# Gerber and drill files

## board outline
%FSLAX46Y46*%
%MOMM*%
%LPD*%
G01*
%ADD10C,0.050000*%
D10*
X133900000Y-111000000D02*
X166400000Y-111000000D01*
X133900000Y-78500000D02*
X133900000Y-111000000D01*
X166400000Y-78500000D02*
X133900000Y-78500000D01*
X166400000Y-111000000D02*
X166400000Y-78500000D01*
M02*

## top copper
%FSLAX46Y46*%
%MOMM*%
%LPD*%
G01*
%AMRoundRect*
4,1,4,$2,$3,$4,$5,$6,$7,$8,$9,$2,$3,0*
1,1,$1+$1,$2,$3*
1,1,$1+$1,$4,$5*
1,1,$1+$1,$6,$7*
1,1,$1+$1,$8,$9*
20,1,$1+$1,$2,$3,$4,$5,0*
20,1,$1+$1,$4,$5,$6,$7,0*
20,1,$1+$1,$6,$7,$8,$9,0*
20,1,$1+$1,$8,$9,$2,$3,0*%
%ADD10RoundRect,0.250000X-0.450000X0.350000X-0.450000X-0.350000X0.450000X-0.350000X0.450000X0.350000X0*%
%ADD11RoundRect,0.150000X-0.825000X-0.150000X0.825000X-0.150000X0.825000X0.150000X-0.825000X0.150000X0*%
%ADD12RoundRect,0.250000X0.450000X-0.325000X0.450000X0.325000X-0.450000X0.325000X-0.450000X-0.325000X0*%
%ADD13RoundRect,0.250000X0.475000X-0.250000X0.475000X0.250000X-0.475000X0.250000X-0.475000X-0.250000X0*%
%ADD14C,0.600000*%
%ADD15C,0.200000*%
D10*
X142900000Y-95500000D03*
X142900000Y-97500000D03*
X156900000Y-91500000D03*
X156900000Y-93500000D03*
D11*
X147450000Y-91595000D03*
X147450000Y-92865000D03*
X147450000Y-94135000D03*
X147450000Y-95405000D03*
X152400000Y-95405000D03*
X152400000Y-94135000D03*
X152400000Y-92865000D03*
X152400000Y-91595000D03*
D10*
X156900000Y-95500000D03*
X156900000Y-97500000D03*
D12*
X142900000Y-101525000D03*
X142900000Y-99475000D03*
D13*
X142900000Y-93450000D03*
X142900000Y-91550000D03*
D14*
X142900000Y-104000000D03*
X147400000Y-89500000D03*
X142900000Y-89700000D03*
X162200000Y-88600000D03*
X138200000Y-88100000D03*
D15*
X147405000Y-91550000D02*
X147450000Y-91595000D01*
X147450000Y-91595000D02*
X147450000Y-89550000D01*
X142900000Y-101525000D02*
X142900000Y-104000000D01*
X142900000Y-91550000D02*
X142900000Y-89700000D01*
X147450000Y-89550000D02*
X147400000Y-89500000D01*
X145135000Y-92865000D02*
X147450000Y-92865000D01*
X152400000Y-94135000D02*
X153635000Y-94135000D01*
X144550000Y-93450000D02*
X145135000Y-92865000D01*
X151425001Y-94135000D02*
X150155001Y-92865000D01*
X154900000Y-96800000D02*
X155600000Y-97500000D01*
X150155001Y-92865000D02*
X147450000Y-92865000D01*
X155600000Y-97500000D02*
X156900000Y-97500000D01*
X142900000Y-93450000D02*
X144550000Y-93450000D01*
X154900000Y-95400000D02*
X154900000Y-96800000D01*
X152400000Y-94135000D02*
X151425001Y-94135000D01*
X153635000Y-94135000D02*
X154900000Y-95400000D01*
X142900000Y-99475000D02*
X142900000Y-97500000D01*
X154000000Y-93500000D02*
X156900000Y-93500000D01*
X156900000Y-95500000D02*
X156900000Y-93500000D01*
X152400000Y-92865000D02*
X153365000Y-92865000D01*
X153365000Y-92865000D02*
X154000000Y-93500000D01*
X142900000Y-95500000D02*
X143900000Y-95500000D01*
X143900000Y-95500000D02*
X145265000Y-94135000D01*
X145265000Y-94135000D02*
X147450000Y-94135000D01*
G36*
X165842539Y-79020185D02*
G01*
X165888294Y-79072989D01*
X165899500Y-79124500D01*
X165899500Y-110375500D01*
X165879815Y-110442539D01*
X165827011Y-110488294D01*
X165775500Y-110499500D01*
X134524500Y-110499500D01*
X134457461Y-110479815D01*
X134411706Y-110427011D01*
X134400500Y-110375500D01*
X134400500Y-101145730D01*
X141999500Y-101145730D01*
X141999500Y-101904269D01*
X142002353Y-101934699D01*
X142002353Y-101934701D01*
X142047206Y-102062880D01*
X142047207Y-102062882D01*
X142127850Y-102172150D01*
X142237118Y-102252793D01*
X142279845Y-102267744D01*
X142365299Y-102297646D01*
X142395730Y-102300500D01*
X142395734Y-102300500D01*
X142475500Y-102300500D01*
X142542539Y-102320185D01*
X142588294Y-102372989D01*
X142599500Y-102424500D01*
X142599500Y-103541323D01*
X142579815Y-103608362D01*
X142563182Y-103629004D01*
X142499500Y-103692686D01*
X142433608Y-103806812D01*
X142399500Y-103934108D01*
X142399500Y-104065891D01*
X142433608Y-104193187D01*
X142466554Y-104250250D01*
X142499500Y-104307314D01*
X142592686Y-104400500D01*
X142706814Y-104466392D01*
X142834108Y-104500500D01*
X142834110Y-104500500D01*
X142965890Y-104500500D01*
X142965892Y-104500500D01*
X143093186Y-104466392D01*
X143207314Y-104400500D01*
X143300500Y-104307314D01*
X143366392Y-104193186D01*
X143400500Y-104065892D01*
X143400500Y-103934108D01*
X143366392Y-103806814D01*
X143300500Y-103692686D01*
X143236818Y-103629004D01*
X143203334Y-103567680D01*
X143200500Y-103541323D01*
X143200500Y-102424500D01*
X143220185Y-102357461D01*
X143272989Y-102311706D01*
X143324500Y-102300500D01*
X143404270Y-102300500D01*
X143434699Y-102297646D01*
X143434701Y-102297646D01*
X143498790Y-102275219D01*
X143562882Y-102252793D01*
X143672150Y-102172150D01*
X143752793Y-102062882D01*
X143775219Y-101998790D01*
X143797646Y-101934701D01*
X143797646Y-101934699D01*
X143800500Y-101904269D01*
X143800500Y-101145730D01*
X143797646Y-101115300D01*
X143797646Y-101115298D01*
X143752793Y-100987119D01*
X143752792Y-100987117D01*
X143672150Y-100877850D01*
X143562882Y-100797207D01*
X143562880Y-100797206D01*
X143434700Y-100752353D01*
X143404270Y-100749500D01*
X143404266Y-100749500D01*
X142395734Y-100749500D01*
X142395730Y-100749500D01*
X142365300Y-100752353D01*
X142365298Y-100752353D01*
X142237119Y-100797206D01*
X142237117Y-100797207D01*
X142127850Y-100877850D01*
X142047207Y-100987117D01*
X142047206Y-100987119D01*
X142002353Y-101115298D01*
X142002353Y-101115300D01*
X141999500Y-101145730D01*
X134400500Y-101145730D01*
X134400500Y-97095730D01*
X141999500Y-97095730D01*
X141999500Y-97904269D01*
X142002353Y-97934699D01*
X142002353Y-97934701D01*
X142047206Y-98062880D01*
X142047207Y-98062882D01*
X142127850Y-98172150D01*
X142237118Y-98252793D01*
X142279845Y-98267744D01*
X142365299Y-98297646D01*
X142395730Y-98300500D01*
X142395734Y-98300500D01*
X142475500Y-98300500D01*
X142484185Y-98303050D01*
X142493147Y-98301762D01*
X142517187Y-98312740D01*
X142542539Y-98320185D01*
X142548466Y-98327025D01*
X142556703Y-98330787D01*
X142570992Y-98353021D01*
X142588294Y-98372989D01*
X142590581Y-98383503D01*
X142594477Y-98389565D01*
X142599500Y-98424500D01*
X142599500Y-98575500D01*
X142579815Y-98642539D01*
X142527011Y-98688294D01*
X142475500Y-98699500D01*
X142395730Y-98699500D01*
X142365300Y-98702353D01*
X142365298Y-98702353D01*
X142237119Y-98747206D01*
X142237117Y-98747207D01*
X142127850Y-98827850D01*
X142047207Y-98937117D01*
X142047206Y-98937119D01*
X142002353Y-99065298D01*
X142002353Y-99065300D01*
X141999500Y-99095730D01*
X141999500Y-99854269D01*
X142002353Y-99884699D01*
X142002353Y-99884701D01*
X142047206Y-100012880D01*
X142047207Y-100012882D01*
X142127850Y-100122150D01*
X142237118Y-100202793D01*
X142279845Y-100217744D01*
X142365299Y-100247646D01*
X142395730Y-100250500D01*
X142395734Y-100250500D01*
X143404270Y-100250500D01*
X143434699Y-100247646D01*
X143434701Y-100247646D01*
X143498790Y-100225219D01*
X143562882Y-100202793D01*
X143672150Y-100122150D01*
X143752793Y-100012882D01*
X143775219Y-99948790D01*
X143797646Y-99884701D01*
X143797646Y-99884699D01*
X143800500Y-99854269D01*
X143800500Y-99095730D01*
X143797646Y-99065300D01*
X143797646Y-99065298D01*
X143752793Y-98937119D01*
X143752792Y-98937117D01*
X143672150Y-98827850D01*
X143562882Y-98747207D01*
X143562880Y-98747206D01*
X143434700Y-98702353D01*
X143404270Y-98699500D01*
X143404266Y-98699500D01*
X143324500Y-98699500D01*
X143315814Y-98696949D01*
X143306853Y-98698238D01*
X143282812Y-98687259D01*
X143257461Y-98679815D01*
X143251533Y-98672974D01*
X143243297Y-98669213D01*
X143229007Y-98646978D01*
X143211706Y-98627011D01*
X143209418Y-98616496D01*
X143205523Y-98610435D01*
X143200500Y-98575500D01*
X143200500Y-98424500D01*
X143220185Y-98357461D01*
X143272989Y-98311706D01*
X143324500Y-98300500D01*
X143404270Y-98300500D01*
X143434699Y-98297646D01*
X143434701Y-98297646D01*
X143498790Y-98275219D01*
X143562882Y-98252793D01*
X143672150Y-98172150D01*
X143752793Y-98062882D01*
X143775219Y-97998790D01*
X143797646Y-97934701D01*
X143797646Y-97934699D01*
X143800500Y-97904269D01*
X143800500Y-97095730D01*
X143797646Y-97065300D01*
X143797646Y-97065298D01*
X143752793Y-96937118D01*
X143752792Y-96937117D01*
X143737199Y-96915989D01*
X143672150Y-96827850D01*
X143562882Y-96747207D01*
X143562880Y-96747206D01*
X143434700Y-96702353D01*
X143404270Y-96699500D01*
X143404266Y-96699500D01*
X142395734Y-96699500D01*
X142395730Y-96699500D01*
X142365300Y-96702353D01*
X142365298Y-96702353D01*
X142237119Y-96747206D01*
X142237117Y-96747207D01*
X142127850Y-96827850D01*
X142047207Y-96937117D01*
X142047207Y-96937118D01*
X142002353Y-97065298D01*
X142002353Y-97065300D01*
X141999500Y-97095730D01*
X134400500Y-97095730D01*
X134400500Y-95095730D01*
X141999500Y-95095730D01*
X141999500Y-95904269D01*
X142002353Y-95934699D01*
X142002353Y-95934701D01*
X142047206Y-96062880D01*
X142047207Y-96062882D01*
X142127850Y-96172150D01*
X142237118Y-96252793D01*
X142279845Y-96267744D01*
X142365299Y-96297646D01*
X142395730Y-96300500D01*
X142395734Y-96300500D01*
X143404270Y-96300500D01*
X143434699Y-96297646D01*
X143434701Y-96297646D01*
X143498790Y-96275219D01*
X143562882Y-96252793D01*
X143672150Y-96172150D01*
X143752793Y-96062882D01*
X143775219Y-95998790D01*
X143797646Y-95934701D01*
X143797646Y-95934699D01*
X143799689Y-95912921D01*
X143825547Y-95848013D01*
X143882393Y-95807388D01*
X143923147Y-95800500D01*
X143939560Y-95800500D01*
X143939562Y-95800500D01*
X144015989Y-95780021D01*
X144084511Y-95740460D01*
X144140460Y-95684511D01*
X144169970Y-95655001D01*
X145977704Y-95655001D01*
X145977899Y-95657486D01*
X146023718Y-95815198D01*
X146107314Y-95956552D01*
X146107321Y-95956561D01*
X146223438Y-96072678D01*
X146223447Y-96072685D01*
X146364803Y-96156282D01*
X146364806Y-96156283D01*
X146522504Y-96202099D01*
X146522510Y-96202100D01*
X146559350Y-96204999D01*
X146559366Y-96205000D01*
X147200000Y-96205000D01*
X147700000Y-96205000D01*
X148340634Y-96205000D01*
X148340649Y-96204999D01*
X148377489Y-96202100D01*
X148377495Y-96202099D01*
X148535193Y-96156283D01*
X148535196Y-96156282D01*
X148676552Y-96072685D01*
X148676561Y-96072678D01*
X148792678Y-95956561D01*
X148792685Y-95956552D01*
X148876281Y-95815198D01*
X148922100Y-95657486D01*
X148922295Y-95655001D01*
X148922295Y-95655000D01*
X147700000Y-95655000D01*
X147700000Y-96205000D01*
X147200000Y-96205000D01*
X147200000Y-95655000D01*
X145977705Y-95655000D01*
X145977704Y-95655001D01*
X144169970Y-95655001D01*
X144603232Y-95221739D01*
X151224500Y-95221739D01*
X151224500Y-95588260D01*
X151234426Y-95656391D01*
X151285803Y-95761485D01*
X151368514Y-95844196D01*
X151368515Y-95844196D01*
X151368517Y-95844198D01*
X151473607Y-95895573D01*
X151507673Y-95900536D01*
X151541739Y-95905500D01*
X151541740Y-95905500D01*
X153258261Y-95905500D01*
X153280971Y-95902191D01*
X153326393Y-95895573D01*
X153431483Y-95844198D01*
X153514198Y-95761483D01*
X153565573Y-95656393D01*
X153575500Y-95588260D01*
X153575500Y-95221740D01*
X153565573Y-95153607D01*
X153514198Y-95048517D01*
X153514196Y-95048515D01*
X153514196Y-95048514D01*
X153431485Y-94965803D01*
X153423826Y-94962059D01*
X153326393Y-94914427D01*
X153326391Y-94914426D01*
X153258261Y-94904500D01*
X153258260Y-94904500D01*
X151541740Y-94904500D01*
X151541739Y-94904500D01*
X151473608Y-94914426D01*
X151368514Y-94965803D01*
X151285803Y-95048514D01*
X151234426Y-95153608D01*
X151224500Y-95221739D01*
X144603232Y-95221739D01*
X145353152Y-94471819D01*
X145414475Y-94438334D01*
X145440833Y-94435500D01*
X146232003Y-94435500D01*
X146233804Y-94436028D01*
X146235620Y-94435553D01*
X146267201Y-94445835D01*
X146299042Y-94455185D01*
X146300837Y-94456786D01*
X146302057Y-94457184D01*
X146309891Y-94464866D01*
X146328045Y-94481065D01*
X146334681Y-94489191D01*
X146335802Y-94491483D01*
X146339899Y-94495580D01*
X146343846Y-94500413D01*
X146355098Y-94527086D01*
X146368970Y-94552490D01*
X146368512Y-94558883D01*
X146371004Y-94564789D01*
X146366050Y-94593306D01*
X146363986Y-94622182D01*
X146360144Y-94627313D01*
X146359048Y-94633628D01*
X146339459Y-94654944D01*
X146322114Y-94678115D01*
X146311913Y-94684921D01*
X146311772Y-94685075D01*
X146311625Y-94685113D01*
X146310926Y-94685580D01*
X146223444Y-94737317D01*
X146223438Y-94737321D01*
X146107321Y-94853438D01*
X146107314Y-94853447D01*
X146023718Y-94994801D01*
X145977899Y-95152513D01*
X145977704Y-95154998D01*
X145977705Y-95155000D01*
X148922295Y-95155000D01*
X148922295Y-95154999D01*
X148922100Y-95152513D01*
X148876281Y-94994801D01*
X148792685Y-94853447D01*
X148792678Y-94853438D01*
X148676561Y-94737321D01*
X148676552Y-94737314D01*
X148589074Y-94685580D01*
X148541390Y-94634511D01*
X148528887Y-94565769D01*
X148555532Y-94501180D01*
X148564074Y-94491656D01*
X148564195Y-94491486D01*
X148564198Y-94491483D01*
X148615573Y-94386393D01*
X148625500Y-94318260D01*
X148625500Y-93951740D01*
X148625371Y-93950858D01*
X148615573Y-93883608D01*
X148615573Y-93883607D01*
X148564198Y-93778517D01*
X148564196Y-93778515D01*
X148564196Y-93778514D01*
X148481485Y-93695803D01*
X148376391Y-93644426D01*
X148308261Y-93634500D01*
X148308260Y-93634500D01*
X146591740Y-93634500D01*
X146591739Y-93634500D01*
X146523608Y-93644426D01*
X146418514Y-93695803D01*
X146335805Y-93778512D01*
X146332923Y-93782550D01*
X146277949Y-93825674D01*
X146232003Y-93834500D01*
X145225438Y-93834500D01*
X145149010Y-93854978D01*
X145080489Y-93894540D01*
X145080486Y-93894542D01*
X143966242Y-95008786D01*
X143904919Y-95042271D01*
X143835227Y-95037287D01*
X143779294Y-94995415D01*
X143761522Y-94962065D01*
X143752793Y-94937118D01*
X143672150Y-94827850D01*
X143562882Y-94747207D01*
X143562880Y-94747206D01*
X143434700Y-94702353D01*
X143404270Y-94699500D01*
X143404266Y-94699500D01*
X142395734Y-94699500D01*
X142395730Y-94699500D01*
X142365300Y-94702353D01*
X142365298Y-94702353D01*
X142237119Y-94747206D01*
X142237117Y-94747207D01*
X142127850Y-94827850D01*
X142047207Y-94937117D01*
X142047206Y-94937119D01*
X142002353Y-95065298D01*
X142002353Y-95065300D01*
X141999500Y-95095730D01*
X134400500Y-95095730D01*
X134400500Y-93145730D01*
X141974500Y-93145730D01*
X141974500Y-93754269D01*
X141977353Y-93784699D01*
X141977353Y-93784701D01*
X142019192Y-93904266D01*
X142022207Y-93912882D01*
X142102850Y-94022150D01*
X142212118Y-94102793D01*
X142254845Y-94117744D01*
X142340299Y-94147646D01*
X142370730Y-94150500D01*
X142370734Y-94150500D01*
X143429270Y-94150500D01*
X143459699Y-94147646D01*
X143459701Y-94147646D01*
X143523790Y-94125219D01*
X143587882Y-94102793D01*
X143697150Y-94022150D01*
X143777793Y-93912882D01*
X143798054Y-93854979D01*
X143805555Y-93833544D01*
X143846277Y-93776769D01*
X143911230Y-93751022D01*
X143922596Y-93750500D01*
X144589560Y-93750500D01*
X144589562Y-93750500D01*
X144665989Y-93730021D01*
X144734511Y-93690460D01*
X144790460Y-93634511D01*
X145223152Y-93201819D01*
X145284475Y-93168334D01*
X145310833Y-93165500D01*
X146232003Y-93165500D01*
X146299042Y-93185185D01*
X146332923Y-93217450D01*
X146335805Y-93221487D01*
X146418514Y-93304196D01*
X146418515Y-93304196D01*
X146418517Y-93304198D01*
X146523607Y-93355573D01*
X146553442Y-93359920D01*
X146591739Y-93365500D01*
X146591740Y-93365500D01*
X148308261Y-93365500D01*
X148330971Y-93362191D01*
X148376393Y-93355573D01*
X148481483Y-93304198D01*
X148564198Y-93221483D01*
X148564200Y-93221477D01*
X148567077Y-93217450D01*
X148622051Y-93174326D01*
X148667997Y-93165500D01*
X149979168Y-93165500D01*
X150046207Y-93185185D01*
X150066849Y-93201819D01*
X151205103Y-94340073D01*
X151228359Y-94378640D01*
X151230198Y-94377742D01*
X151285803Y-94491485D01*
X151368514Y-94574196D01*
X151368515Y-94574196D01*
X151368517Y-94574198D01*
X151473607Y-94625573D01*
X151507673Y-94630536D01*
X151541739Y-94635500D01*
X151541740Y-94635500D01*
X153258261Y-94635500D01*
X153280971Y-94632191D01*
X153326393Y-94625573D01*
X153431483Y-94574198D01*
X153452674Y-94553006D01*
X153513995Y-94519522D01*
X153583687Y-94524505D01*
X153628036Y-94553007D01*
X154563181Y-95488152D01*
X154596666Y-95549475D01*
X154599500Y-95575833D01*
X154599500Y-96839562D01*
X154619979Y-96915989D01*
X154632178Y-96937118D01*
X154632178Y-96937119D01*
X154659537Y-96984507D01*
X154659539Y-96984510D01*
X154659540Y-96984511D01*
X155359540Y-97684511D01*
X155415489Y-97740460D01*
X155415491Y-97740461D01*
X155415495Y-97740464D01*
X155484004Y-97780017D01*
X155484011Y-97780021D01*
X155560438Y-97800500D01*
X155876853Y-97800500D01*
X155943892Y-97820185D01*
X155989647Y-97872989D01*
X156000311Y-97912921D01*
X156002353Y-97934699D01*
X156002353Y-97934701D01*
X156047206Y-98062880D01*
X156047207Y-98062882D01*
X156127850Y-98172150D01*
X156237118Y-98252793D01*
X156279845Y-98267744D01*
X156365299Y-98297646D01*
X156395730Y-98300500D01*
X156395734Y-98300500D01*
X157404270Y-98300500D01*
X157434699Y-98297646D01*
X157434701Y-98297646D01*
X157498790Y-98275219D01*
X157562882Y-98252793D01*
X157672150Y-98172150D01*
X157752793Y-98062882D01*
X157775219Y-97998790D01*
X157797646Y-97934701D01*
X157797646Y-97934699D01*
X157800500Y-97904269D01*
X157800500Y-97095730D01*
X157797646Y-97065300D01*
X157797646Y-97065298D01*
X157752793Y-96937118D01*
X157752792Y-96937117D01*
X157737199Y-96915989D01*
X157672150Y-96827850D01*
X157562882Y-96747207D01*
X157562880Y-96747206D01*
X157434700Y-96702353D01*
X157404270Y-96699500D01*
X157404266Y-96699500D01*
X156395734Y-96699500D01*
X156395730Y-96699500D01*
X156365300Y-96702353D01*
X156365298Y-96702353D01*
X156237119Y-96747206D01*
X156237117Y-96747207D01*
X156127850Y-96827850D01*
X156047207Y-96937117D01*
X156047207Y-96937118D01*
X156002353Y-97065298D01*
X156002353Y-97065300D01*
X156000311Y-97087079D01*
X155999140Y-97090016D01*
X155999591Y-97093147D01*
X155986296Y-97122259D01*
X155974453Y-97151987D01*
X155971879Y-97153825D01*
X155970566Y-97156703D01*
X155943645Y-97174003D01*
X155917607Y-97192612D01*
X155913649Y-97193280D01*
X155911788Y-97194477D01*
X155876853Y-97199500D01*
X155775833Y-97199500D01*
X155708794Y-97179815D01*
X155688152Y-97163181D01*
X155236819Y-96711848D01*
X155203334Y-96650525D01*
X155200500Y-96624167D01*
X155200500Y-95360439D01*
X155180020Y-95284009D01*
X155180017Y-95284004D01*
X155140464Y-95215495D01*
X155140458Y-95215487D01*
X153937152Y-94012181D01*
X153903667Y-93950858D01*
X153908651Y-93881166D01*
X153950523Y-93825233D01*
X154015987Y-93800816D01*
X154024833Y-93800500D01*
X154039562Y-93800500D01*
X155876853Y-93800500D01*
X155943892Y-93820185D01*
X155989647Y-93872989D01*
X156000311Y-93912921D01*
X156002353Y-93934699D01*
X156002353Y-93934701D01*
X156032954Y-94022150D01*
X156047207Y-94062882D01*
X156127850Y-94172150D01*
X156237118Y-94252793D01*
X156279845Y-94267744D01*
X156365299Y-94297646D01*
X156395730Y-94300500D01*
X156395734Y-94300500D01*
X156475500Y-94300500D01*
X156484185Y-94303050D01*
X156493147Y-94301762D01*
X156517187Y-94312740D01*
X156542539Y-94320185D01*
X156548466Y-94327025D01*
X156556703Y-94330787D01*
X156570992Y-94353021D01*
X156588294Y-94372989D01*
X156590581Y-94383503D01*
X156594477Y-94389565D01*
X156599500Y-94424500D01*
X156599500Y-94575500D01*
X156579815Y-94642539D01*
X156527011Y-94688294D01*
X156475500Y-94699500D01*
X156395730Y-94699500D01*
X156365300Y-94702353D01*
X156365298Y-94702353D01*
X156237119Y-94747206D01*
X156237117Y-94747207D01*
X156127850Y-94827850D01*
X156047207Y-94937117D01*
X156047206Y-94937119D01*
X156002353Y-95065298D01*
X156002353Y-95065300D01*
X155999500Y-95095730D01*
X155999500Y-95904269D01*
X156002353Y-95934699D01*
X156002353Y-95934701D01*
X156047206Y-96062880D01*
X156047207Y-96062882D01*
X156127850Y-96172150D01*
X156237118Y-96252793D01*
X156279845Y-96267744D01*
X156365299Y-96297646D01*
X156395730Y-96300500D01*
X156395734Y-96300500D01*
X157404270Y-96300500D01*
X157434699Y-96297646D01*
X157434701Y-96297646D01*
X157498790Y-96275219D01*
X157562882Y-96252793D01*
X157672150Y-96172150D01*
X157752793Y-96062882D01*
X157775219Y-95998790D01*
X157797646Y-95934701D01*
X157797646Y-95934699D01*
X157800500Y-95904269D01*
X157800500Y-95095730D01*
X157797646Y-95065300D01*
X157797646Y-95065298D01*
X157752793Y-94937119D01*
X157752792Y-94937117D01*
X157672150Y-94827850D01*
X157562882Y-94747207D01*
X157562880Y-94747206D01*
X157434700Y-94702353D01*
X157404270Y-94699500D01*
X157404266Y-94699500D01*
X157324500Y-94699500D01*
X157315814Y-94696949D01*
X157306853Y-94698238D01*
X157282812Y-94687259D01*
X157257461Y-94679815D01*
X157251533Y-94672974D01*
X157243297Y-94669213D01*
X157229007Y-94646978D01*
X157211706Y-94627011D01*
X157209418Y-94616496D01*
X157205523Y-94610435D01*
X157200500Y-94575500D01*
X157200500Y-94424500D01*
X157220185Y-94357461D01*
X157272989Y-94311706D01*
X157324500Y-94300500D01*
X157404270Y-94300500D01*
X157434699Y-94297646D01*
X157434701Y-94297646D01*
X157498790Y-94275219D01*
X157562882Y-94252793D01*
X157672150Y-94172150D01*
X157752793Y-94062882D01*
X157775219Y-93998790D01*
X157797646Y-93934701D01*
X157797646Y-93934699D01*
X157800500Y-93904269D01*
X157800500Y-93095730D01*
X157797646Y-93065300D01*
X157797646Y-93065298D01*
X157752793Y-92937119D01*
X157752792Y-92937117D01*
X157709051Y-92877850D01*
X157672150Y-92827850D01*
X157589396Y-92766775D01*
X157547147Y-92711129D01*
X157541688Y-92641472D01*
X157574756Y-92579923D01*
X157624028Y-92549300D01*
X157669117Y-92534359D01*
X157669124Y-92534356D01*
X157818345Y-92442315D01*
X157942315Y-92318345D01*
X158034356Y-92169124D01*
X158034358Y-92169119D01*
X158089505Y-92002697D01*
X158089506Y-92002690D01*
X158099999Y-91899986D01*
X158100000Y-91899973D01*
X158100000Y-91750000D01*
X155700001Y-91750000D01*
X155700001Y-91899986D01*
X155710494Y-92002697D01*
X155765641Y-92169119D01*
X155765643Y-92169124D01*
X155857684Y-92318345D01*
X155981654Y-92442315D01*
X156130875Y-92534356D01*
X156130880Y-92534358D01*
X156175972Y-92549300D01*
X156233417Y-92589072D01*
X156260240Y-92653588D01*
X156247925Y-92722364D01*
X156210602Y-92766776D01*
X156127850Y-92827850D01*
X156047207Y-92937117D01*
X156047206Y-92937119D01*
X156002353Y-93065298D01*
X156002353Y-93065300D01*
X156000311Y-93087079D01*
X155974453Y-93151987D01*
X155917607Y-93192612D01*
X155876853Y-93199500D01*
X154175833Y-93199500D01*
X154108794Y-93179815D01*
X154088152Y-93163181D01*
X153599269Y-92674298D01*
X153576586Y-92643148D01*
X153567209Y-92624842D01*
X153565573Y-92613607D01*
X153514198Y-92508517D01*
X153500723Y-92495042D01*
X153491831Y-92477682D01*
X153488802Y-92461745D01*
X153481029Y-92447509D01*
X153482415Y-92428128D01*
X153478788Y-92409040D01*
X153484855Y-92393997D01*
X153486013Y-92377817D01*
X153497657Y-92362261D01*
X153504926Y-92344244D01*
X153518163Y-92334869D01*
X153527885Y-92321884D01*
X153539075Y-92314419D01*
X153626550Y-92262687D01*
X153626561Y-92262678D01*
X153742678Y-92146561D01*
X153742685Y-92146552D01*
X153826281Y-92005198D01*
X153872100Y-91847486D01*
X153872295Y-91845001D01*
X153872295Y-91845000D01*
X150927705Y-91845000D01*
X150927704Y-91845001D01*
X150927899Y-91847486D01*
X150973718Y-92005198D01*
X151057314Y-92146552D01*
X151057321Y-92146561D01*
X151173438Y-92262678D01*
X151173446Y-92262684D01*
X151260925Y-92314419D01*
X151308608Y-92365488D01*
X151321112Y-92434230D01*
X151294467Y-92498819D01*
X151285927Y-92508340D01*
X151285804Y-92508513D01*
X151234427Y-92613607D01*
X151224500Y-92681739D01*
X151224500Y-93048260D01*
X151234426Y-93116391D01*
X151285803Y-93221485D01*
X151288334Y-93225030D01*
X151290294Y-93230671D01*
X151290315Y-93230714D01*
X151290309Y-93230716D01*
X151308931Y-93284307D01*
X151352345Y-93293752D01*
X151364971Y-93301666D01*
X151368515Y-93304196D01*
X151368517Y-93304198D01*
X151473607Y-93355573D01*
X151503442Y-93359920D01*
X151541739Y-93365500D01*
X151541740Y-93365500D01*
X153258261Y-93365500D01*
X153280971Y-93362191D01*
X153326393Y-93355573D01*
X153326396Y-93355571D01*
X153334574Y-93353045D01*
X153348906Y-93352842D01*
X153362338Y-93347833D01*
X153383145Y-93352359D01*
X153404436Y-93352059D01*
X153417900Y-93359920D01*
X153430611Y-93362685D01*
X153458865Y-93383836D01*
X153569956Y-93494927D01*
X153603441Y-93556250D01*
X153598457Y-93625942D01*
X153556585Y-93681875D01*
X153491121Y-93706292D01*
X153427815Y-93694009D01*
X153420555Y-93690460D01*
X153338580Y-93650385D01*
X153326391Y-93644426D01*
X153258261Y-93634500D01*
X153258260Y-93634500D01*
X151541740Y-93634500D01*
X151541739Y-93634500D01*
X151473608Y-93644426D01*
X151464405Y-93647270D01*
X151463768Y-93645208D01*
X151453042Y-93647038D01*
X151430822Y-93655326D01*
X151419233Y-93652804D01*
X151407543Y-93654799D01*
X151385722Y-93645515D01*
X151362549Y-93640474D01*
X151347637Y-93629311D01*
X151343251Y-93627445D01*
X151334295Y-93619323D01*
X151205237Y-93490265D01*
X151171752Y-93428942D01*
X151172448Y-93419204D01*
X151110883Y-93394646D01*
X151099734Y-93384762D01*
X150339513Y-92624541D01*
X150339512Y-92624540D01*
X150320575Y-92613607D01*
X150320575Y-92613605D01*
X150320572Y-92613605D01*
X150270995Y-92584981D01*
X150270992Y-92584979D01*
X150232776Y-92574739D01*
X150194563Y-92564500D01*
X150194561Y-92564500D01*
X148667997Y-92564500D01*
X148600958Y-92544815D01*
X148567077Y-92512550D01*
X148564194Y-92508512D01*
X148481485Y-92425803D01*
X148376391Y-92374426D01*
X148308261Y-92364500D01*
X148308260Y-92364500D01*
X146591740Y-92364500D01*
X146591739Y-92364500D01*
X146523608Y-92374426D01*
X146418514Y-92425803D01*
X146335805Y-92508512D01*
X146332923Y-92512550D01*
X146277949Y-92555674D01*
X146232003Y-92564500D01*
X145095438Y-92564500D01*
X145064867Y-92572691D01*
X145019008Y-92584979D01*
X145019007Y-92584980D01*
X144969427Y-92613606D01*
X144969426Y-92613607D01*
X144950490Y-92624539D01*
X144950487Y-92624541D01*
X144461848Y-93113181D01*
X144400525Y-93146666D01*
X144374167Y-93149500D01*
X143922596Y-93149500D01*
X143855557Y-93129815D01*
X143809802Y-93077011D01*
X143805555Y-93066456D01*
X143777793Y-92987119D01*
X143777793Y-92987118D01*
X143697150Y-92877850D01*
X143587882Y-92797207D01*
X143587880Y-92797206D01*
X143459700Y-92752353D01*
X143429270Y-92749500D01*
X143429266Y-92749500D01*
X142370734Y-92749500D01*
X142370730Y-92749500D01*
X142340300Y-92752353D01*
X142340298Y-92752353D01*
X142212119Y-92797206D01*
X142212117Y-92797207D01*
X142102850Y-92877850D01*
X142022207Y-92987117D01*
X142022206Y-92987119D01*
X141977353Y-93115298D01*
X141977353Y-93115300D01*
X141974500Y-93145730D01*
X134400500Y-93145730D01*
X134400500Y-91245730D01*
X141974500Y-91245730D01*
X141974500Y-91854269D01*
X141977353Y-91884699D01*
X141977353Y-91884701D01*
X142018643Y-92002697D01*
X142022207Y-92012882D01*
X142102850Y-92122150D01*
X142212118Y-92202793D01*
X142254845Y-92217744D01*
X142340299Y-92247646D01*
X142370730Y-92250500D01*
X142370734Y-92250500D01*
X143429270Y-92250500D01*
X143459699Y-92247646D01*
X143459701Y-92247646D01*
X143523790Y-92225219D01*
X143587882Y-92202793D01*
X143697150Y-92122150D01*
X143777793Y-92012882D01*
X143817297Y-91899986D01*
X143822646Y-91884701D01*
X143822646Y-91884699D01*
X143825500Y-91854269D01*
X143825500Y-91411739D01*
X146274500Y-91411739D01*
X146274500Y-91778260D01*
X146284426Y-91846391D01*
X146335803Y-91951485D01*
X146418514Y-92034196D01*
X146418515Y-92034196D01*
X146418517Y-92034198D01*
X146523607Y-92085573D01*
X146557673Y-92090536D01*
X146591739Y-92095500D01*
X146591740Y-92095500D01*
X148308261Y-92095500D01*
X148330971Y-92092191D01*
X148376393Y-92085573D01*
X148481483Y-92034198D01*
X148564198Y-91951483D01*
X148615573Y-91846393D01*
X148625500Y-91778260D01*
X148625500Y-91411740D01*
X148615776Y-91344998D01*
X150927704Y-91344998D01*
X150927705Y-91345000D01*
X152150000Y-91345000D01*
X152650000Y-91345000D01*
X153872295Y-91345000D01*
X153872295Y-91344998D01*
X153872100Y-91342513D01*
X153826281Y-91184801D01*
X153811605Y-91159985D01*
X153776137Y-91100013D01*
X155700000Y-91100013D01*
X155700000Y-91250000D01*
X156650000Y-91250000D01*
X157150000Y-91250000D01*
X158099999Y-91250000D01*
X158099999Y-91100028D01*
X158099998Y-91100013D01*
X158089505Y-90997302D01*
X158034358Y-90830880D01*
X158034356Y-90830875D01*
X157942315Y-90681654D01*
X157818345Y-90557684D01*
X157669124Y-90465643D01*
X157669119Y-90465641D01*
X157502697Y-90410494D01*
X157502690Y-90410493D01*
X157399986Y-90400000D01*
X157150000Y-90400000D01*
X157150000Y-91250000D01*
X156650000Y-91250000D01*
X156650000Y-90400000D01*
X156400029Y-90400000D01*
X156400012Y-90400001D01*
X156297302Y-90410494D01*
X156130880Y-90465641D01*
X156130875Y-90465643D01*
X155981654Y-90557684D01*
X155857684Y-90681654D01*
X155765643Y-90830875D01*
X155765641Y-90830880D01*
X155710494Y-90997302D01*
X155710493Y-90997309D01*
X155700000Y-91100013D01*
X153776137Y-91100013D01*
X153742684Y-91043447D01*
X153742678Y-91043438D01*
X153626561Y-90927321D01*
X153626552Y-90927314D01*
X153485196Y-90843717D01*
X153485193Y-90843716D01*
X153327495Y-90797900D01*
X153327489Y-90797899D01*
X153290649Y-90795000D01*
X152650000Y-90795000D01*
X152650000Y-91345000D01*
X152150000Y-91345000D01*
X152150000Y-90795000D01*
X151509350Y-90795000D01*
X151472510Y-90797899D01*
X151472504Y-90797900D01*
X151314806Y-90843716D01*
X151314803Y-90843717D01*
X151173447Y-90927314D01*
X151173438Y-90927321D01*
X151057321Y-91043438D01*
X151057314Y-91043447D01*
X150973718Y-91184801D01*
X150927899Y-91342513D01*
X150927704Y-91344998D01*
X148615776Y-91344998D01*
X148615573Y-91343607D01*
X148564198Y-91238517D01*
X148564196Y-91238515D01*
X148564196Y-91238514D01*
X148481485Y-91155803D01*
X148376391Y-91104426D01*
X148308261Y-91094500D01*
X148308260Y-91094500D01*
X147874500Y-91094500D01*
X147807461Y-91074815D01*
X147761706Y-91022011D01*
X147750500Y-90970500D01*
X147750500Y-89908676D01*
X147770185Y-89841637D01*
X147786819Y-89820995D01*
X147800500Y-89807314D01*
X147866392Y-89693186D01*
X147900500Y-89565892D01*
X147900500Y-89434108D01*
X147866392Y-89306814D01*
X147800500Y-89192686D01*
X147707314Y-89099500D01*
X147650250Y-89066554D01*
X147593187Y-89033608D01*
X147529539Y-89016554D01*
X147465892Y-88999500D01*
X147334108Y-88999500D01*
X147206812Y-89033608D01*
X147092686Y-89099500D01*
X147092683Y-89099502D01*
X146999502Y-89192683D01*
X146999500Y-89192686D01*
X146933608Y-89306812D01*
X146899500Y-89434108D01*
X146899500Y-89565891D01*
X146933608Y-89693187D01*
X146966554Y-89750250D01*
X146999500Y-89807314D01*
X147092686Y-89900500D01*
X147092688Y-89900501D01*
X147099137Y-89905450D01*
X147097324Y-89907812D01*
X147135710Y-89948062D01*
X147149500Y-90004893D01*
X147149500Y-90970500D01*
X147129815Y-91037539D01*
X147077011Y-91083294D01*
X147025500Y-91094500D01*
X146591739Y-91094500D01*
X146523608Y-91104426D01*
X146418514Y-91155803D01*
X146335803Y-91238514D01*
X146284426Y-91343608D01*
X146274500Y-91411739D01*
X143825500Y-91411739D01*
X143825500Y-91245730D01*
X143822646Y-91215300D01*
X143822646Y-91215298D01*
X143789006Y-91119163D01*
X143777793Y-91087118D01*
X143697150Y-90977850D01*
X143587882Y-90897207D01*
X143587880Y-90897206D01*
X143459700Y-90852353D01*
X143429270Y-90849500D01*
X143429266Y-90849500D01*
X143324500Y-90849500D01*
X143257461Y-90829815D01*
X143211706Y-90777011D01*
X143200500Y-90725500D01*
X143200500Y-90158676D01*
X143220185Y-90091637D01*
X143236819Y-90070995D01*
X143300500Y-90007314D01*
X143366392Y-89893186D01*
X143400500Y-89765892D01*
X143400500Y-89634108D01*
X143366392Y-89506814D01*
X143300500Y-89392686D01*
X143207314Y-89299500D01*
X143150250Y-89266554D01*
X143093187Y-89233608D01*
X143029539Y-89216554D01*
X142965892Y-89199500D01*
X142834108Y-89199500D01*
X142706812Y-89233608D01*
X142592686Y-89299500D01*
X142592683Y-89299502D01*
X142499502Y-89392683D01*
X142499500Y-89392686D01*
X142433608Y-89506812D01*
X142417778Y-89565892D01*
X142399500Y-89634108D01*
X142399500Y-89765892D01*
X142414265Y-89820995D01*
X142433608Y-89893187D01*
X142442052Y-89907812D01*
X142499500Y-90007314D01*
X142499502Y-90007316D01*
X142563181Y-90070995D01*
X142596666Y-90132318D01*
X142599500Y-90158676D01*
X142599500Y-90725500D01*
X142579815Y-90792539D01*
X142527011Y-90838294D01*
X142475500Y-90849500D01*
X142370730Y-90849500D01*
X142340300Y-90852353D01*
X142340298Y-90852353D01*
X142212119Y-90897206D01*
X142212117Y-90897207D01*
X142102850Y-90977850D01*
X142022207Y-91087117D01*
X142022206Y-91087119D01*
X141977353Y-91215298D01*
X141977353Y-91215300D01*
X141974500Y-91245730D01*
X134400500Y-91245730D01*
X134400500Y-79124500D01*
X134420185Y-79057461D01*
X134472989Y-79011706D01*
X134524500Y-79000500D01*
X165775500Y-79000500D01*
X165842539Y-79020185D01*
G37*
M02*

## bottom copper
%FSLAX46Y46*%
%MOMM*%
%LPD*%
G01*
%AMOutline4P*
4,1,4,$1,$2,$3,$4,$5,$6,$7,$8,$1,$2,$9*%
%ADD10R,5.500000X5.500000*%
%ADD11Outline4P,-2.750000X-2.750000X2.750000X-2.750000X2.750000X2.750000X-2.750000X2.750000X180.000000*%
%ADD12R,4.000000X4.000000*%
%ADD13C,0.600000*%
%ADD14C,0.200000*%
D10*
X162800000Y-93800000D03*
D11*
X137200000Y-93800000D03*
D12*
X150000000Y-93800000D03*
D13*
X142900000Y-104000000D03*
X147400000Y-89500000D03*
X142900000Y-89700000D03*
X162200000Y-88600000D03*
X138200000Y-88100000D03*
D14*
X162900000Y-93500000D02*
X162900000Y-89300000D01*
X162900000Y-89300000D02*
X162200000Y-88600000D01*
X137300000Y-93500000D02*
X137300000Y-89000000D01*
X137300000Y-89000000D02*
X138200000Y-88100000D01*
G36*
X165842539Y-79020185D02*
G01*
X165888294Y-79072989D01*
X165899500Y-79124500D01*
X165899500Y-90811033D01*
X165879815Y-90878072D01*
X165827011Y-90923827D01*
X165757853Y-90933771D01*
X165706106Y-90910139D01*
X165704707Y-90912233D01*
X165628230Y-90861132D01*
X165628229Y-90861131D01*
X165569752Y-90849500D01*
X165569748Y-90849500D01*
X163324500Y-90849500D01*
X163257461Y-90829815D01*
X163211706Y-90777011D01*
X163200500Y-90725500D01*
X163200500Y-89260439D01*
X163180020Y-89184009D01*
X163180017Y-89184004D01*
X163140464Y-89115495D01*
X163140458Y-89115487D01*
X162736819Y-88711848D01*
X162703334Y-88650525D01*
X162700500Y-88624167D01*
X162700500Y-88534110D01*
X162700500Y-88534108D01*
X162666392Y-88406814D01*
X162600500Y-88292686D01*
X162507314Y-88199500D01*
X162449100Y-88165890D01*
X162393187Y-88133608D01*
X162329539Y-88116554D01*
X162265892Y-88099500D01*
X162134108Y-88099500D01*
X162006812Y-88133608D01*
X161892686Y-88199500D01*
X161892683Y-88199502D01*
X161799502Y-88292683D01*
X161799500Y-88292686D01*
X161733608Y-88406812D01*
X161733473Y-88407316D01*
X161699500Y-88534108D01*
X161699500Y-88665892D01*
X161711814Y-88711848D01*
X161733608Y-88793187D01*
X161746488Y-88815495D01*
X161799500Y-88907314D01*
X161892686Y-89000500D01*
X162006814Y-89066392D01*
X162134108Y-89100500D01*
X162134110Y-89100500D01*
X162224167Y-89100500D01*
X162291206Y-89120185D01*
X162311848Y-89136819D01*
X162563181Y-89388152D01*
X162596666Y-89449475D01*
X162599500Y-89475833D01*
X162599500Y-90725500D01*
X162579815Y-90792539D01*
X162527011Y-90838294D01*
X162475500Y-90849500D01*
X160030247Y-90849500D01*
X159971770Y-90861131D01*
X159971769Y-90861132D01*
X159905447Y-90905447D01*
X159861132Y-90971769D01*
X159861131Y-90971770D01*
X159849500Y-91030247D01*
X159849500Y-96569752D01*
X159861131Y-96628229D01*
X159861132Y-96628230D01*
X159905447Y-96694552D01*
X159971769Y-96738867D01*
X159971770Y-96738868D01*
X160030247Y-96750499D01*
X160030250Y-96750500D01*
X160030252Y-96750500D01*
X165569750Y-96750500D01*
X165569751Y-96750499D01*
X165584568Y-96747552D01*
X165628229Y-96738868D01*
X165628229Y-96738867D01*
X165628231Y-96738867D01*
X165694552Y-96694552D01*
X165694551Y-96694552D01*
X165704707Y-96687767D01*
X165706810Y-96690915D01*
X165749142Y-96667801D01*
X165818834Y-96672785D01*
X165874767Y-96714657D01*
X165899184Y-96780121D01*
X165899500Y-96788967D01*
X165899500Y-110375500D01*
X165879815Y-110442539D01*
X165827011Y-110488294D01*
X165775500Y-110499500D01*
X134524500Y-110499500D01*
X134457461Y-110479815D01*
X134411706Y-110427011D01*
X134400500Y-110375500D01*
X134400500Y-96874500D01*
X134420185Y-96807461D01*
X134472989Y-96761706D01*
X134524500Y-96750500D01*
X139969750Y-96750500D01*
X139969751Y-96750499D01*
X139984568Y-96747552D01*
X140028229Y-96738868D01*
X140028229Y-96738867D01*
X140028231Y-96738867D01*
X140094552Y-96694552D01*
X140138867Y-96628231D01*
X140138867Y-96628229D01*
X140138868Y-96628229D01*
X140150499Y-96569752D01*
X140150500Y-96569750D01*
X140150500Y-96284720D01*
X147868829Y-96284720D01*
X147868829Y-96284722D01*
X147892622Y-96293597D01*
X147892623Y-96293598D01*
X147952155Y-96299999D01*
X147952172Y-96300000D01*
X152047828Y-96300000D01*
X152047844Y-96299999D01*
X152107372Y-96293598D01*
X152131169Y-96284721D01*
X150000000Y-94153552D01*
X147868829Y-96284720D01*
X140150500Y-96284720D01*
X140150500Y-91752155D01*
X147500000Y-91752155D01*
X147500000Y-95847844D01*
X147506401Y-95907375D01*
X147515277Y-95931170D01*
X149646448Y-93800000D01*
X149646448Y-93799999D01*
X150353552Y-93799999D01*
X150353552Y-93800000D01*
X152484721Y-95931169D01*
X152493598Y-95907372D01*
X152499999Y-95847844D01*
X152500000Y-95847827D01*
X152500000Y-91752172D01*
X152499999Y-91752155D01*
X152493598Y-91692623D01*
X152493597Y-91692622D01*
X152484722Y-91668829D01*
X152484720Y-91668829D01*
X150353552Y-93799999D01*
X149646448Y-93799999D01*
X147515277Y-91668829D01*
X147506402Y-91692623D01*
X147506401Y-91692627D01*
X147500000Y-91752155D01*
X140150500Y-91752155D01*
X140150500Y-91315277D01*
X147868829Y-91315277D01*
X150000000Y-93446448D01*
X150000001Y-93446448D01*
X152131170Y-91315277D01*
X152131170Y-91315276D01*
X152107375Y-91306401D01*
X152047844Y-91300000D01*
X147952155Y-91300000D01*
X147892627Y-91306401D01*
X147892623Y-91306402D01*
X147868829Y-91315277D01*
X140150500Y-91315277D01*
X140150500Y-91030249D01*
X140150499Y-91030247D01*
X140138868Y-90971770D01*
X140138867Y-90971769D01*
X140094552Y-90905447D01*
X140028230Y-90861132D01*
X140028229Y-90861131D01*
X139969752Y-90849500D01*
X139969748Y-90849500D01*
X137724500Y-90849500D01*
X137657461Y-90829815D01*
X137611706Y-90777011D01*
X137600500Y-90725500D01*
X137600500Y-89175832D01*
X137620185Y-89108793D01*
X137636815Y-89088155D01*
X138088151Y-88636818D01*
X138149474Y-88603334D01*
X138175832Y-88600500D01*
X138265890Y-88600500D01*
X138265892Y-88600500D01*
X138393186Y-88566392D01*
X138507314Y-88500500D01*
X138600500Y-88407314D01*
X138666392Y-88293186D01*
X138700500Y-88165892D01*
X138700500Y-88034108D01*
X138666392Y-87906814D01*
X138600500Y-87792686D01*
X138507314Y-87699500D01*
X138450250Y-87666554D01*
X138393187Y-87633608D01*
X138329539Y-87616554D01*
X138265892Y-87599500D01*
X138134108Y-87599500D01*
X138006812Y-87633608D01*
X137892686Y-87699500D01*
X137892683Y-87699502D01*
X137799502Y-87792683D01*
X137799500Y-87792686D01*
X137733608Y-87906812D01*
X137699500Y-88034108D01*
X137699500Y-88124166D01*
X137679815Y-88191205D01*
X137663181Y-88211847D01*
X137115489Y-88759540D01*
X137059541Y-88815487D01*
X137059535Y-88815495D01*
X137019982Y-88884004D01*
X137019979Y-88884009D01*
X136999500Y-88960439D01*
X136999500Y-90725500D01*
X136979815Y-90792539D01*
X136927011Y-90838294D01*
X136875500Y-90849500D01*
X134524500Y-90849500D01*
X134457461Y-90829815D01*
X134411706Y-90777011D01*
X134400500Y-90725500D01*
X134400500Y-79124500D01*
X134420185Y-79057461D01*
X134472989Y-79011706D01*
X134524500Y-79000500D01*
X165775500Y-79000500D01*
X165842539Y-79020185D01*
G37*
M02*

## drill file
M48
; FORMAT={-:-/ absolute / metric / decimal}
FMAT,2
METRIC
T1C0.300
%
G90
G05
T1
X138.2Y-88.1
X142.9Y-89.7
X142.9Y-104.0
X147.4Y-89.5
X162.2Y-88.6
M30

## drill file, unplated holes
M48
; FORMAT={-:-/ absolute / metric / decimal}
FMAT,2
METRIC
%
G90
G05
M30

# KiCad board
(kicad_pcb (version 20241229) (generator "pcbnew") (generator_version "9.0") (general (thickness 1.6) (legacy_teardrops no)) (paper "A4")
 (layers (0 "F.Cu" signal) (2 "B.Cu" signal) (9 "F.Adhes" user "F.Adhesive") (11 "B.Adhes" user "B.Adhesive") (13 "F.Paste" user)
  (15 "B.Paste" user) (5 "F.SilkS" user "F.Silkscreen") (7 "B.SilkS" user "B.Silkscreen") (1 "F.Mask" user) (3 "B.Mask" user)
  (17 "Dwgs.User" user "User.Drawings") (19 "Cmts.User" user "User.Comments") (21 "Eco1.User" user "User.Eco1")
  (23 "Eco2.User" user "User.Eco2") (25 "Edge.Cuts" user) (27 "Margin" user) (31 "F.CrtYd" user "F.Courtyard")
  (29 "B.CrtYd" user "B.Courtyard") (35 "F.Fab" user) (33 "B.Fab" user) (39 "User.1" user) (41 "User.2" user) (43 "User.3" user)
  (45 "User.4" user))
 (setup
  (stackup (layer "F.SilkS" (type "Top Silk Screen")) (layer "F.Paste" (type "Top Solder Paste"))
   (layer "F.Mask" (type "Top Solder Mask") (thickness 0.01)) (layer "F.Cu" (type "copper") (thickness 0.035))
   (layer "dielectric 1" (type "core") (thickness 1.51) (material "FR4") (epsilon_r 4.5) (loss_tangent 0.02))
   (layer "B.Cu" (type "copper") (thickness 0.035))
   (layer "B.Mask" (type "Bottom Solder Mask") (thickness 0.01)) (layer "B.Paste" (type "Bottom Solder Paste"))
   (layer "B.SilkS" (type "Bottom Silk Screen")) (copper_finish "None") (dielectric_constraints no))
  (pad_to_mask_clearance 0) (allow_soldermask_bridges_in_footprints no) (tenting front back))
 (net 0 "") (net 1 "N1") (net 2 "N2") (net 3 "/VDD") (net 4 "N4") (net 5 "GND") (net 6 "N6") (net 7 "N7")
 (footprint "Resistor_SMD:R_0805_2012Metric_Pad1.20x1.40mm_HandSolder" (layer "F.Cu") (at 142.9 96.5 -90)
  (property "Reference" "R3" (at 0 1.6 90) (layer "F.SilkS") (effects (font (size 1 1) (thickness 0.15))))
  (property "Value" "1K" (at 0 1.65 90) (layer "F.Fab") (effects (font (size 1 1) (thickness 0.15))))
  (pad "1" smd roundrect (at -1 0 270) (size 1.2 1.4) (layers "F.Cu" "F.Mask" "F.Paste") (roundrect_rratio 0.208333) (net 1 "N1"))
  (pad "2" smd roundrect (at 1 0 270) (size 1.2 1.4) (layers "F.Cu" "F.Mask" "F.Paste") (roundrect_rratio 0.208333) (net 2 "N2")))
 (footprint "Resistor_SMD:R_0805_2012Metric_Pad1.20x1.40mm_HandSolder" (layer "F.Cu") (at 156.9 92.5 -90)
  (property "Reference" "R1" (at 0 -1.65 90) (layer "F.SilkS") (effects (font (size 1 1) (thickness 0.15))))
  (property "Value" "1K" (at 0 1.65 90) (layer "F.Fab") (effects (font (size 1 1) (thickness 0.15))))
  (pad "1" smd roundrect (at -1 0 270) (size 1.2 1.4) (layers "F.Cu" "F.Mask" "F.Paste") (roundrect_rratio 0.208333) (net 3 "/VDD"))
  (pad "2" smd roundrect (at 1 0 270) (size 1.2 1.4) (layers "F.Cu" "F.Mask" "F.Paste") (roundrect_rratio 0.208333) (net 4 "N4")))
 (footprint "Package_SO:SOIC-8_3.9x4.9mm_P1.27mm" (layer "F.Cu") (at 149.925 93.5)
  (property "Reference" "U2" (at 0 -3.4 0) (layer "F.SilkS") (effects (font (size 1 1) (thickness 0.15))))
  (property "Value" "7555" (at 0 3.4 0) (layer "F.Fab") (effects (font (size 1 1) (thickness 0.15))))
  (pad "1" smd roundrect (at -2.475 -1.905) (size 1.95 0.6) (layers "F.Cu" "F.Mask" "F.Paste") (roundrect_rratio 0.25) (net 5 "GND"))
  (pad "2" smd roundrect (at -2.475 -0.635) (size 1.95 0.6) (layers "F.Cu" "F.Mask" "F.Paste") (roundrect_rratio 0.25) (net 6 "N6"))
  (pad "3" smd roundrect (at -2.475 0.635) (size 1.95 0.6) (layers "F.Cu" "F.Mask" "F.Paste") (roundrect_rratio 0.25) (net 1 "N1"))
  (pad "4" smd roundrect (at -2.475 1.905) (size 1.95 0.6) (layers "F.Cu" "F.Mask" "F.Paste") (roundrect_rratio 0.25) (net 3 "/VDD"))
  (pad "5" smd roundrect (at 2.475 1.905) (size 1.95 0.6) (layers "F.Cu" "F.Mask" "F.Paste") (roundrect_rratio 0.25) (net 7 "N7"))
  (pad "6" smd roundrect (at 2.475 0.635) (size 1.95 0.6) (layers "F.Cu" "F.Mask" "F.Paste") (roundrect_rratio 0.25) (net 6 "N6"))
  (pad "7" smd roundrect (at 2.475 -0.635) (size 1.95 0.6) (layers "F.Cu" "F.Mask" "F.Paste") (roundrect_rratio 0.25) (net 4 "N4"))
  (pad "8" smd roundrect (at 2.475 -1.905) (size 1.95 0.6) (layers "F.Cu" "F.Mask" "F.Paste") (roundrect_rratio 0.25) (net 3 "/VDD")))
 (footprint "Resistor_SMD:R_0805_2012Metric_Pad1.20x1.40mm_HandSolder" (layer "F.Cu") (at 156.9 96.5 -90)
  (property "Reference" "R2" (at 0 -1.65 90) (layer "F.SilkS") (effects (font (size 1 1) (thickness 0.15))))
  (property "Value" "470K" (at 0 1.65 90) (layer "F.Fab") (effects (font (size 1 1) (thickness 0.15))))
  (pad "1" smd roundrect (at -1 0 270) (size 1.2 1.4) (layers "F.Cu" "F.Mask" "F.Paste") (roundrect_rratio 0.208333) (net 4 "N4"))
  (pad "2" smd roundrect (at 1 0 270) (size 1.2 1.4) (layers "F.Cu" "F.Mask" "F.Paste") (roundrect_rratio 0.208333) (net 6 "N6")))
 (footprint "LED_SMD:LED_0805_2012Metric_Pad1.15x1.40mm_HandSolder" (layer "F.Cu") (at 142.9 100.5 90)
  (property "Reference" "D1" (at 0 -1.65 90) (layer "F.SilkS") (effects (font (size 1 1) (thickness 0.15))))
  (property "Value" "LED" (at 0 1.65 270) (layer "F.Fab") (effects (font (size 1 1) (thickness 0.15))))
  (pad "1" smd roundrect (at -1.025 0 90) (size 1.15 1.4) (layers "F.Cu" "F.Mask" "F.Paste") (roundrect_rratio 0.217391) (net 5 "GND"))
  (pad "2" smd roundrect (at 1.025 0 90) (size 1.15 1.4) (layers "F.Cu" "F.Mask" "F.Paste") (roundrect_rratio 0.217391) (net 2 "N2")))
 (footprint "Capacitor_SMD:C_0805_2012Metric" (layer "F.Cu") (at 142.9 92.5 90)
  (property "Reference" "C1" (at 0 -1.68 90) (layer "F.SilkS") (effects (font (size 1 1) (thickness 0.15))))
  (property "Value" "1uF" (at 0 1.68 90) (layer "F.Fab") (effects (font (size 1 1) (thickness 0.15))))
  (pad "1" smd roundrect (at -0.95 0 90) (size 1 1.45) (layers "F.Cu" "F.Mask" "F.Paste") (roundrect_rratio 0.25) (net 6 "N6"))
  (pad "2" smd roundrect (at 0.95 0 90) (size 1 1.45) (layers "F.Cu" "F.Mask" "F.Paste") (roundrect_rratio 0.25) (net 5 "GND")))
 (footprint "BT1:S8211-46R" (layer "B.Cu") (at 150 93.8 180)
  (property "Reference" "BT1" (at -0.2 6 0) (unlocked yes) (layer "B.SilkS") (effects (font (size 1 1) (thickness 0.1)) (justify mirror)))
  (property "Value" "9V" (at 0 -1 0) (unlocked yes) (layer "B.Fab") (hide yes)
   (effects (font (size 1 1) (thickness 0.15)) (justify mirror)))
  (pad "1" smd rect (at -12.8 0 180) (size 5.5 5.5) (layers "B.Cu" "B.Mask" "B.Paste") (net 3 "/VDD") (thermal_bridge_angle 45))
  (pad "1" smd trapezoid (at 12.8 0 180) (size 5.5 5.5) (layers "B.Cu" "B.Mask" "B.Paste") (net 3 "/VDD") (thermal_bridge_angle 45))
  (pad "2" smd rect (at 0 0 90) (size 4 4) (layers "B.Cu" "B.Mask" "B.Paste") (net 5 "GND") (thermal_bridge_angle 45)))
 (gr_line (start 133.9 111) (end 166.4 111) (stroke (width 0.05) (type default)) (layer "Edge.Cuts"))
 (gr_line (start 133.9 78.5) (end 133.9 111) (stroke (width 0.05) (type default)) (layer "Edge.Cuts"))
 (gr_line (start 166.4 78.5) (end 133.9 78.5) (stroke (width 0.05) (type default)) (layer "Edge.Cuts"))
 (gr_line (start 166.4 111) (end 166.4 78.5) (stroke (width 0.05) (type default)) (layer "Edge.Cuts"))
 (segment (start 147.405 91.55) (end 147.45 91.595) (width 0.2) (layer "F.Cu") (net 5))
 (segment (start 147.45 91.595) (end 147.45 89.55) (width 0.2) (layer "F.Cu") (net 5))
 (segment (start 142.9 101.525) (end 142.9 104) (width 0.2) (layer "F.Cu") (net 5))
 (segment (start 142.9 91.55) (end 142.9 89.7) (width 0.2) (layer "F.Cu") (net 5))
 (segment (start 147.45 89.55) (end 147.4 89.5) (width 0.2) (layer "F.Cu") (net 5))
 (via (at 142.9 104) (size 0.6) (drill 0.3) (layers "F.Cu" "B.Cu") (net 5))
 (via (at 147.4 89.5) (size 0.6) (drill 0.3) (layers "F.Cu" "B.Cu") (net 5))
 (via (at 142.9 89.7) (size 0.6) (drill 0.3) (layers "F.Cu" "B.Cu") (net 5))
 (via (at 162.2 88.6) (size 0.6) (drill 0.3) (layers "F.Cu" "B.Cu") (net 3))
 (via (at 138.2 88.1) (size 0.6) (drill 0.3) (layers "F.Cu" "B.Cu") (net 3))
 (segment (start 162.9 93.5) (end 162.9 89.3) (width 0.2) (layer "B.Cu") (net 3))
 (segment (start 162.9 89.3) (end 162.2 88.6) (width 0.2) (layer "B.Cu") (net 3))
 (segment (start 137.3 93.5) (end 137.3 89) (width 0.2) (layer "B.Cu") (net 3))
 (segment (start 137.3 89) (end 138.2 88.1) (width 0.2) (layer "B.Cu") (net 3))
 (segment (start 145.135 92.865) (end 147.45 92.865) (width 0.2) (layer "F.Cu") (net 6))
 (segment (start 152.4 94.135) (end 153.635 94.135) (width 0.2) (layer "F.Cu") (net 6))
 (segment (start 144.55 93.45) (end 145.135 92.865) (width 0.2) (layer "F.Cu") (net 6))
 (segment (start 151.425001 94.135) (end 150.155001 92.865) (width 0.2) (layer "F.Cu") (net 6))
 (segment (start 154.9 96.8) (end 155.6 97.5) (width 0.2) (layer "F.Cu") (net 6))
 (segment (start 150.155001 92.865) (end 147.45 92.865) (width 0.2) (layer "F.Cu") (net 6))
 (segment (start 155.6 97.5) (end 156.9 97.5) (width 0.2) (layer "F.Cu") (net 6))
 (segment (start 142.9 93.45) (end 144.55 93.45) (width 0.2) (layer "F.Cu") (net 6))
 (segment (start 154.9 95.4) (end 154.9 96.8) (width 0.2) (layer "F.Cu") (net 6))
 (segment (start 152.4 94.135) (end 151.425001 94.135) (width 0.2) (layer "F.Cu") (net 6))
 (segment (start 153.635 94.135) (end 154.9 95.4) (width 0.2) (layer "F.Cu") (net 6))
 (segment (start 142.9 99.475) (end 142.9 97.5) (width 0.2) (layer "F.Cu") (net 2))
 (segment (start 154 93.5) (end 156.9 93.5) (width 0.2) (layer "F.Cu") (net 4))
 (segment (start 156.9 95.5) (end 156.9 93.5) (width 0.2) (layer "F.Cu") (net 4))
 (segment (start 152.4 92.865) (end 153.365 92.865) (width 0.2) (layer "F.Cu") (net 4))
 (segment (start 153.365 92.865) (end 154 93.5) (width 0.2) (layer "F.Cu") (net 4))
 (segment (start 142.9 95.5) (end 143.9 95.5) (width 0.2) (layer "F.Cu") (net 1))
 (segment (start 143.9 95.5) (end 145.265 94.135) (width 0.2) (layer "F.Cu") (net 1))
 (segment (start 145.265 94.135) (end 147.45 94.135) (width 0.2) (layer "F.Cu") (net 1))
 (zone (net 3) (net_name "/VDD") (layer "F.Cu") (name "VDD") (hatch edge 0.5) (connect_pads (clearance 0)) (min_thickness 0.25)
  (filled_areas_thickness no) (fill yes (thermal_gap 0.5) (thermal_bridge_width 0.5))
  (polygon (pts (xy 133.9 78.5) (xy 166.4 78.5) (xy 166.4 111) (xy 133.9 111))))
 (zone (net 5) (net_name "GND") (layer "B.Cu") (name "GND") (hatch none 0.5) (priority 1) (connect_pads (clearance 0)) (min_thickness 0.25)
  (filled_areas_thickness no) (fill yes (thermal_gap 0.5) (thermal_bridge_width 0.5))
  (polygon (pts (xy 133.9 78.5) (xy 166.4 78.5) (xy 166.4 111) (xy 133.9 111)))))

